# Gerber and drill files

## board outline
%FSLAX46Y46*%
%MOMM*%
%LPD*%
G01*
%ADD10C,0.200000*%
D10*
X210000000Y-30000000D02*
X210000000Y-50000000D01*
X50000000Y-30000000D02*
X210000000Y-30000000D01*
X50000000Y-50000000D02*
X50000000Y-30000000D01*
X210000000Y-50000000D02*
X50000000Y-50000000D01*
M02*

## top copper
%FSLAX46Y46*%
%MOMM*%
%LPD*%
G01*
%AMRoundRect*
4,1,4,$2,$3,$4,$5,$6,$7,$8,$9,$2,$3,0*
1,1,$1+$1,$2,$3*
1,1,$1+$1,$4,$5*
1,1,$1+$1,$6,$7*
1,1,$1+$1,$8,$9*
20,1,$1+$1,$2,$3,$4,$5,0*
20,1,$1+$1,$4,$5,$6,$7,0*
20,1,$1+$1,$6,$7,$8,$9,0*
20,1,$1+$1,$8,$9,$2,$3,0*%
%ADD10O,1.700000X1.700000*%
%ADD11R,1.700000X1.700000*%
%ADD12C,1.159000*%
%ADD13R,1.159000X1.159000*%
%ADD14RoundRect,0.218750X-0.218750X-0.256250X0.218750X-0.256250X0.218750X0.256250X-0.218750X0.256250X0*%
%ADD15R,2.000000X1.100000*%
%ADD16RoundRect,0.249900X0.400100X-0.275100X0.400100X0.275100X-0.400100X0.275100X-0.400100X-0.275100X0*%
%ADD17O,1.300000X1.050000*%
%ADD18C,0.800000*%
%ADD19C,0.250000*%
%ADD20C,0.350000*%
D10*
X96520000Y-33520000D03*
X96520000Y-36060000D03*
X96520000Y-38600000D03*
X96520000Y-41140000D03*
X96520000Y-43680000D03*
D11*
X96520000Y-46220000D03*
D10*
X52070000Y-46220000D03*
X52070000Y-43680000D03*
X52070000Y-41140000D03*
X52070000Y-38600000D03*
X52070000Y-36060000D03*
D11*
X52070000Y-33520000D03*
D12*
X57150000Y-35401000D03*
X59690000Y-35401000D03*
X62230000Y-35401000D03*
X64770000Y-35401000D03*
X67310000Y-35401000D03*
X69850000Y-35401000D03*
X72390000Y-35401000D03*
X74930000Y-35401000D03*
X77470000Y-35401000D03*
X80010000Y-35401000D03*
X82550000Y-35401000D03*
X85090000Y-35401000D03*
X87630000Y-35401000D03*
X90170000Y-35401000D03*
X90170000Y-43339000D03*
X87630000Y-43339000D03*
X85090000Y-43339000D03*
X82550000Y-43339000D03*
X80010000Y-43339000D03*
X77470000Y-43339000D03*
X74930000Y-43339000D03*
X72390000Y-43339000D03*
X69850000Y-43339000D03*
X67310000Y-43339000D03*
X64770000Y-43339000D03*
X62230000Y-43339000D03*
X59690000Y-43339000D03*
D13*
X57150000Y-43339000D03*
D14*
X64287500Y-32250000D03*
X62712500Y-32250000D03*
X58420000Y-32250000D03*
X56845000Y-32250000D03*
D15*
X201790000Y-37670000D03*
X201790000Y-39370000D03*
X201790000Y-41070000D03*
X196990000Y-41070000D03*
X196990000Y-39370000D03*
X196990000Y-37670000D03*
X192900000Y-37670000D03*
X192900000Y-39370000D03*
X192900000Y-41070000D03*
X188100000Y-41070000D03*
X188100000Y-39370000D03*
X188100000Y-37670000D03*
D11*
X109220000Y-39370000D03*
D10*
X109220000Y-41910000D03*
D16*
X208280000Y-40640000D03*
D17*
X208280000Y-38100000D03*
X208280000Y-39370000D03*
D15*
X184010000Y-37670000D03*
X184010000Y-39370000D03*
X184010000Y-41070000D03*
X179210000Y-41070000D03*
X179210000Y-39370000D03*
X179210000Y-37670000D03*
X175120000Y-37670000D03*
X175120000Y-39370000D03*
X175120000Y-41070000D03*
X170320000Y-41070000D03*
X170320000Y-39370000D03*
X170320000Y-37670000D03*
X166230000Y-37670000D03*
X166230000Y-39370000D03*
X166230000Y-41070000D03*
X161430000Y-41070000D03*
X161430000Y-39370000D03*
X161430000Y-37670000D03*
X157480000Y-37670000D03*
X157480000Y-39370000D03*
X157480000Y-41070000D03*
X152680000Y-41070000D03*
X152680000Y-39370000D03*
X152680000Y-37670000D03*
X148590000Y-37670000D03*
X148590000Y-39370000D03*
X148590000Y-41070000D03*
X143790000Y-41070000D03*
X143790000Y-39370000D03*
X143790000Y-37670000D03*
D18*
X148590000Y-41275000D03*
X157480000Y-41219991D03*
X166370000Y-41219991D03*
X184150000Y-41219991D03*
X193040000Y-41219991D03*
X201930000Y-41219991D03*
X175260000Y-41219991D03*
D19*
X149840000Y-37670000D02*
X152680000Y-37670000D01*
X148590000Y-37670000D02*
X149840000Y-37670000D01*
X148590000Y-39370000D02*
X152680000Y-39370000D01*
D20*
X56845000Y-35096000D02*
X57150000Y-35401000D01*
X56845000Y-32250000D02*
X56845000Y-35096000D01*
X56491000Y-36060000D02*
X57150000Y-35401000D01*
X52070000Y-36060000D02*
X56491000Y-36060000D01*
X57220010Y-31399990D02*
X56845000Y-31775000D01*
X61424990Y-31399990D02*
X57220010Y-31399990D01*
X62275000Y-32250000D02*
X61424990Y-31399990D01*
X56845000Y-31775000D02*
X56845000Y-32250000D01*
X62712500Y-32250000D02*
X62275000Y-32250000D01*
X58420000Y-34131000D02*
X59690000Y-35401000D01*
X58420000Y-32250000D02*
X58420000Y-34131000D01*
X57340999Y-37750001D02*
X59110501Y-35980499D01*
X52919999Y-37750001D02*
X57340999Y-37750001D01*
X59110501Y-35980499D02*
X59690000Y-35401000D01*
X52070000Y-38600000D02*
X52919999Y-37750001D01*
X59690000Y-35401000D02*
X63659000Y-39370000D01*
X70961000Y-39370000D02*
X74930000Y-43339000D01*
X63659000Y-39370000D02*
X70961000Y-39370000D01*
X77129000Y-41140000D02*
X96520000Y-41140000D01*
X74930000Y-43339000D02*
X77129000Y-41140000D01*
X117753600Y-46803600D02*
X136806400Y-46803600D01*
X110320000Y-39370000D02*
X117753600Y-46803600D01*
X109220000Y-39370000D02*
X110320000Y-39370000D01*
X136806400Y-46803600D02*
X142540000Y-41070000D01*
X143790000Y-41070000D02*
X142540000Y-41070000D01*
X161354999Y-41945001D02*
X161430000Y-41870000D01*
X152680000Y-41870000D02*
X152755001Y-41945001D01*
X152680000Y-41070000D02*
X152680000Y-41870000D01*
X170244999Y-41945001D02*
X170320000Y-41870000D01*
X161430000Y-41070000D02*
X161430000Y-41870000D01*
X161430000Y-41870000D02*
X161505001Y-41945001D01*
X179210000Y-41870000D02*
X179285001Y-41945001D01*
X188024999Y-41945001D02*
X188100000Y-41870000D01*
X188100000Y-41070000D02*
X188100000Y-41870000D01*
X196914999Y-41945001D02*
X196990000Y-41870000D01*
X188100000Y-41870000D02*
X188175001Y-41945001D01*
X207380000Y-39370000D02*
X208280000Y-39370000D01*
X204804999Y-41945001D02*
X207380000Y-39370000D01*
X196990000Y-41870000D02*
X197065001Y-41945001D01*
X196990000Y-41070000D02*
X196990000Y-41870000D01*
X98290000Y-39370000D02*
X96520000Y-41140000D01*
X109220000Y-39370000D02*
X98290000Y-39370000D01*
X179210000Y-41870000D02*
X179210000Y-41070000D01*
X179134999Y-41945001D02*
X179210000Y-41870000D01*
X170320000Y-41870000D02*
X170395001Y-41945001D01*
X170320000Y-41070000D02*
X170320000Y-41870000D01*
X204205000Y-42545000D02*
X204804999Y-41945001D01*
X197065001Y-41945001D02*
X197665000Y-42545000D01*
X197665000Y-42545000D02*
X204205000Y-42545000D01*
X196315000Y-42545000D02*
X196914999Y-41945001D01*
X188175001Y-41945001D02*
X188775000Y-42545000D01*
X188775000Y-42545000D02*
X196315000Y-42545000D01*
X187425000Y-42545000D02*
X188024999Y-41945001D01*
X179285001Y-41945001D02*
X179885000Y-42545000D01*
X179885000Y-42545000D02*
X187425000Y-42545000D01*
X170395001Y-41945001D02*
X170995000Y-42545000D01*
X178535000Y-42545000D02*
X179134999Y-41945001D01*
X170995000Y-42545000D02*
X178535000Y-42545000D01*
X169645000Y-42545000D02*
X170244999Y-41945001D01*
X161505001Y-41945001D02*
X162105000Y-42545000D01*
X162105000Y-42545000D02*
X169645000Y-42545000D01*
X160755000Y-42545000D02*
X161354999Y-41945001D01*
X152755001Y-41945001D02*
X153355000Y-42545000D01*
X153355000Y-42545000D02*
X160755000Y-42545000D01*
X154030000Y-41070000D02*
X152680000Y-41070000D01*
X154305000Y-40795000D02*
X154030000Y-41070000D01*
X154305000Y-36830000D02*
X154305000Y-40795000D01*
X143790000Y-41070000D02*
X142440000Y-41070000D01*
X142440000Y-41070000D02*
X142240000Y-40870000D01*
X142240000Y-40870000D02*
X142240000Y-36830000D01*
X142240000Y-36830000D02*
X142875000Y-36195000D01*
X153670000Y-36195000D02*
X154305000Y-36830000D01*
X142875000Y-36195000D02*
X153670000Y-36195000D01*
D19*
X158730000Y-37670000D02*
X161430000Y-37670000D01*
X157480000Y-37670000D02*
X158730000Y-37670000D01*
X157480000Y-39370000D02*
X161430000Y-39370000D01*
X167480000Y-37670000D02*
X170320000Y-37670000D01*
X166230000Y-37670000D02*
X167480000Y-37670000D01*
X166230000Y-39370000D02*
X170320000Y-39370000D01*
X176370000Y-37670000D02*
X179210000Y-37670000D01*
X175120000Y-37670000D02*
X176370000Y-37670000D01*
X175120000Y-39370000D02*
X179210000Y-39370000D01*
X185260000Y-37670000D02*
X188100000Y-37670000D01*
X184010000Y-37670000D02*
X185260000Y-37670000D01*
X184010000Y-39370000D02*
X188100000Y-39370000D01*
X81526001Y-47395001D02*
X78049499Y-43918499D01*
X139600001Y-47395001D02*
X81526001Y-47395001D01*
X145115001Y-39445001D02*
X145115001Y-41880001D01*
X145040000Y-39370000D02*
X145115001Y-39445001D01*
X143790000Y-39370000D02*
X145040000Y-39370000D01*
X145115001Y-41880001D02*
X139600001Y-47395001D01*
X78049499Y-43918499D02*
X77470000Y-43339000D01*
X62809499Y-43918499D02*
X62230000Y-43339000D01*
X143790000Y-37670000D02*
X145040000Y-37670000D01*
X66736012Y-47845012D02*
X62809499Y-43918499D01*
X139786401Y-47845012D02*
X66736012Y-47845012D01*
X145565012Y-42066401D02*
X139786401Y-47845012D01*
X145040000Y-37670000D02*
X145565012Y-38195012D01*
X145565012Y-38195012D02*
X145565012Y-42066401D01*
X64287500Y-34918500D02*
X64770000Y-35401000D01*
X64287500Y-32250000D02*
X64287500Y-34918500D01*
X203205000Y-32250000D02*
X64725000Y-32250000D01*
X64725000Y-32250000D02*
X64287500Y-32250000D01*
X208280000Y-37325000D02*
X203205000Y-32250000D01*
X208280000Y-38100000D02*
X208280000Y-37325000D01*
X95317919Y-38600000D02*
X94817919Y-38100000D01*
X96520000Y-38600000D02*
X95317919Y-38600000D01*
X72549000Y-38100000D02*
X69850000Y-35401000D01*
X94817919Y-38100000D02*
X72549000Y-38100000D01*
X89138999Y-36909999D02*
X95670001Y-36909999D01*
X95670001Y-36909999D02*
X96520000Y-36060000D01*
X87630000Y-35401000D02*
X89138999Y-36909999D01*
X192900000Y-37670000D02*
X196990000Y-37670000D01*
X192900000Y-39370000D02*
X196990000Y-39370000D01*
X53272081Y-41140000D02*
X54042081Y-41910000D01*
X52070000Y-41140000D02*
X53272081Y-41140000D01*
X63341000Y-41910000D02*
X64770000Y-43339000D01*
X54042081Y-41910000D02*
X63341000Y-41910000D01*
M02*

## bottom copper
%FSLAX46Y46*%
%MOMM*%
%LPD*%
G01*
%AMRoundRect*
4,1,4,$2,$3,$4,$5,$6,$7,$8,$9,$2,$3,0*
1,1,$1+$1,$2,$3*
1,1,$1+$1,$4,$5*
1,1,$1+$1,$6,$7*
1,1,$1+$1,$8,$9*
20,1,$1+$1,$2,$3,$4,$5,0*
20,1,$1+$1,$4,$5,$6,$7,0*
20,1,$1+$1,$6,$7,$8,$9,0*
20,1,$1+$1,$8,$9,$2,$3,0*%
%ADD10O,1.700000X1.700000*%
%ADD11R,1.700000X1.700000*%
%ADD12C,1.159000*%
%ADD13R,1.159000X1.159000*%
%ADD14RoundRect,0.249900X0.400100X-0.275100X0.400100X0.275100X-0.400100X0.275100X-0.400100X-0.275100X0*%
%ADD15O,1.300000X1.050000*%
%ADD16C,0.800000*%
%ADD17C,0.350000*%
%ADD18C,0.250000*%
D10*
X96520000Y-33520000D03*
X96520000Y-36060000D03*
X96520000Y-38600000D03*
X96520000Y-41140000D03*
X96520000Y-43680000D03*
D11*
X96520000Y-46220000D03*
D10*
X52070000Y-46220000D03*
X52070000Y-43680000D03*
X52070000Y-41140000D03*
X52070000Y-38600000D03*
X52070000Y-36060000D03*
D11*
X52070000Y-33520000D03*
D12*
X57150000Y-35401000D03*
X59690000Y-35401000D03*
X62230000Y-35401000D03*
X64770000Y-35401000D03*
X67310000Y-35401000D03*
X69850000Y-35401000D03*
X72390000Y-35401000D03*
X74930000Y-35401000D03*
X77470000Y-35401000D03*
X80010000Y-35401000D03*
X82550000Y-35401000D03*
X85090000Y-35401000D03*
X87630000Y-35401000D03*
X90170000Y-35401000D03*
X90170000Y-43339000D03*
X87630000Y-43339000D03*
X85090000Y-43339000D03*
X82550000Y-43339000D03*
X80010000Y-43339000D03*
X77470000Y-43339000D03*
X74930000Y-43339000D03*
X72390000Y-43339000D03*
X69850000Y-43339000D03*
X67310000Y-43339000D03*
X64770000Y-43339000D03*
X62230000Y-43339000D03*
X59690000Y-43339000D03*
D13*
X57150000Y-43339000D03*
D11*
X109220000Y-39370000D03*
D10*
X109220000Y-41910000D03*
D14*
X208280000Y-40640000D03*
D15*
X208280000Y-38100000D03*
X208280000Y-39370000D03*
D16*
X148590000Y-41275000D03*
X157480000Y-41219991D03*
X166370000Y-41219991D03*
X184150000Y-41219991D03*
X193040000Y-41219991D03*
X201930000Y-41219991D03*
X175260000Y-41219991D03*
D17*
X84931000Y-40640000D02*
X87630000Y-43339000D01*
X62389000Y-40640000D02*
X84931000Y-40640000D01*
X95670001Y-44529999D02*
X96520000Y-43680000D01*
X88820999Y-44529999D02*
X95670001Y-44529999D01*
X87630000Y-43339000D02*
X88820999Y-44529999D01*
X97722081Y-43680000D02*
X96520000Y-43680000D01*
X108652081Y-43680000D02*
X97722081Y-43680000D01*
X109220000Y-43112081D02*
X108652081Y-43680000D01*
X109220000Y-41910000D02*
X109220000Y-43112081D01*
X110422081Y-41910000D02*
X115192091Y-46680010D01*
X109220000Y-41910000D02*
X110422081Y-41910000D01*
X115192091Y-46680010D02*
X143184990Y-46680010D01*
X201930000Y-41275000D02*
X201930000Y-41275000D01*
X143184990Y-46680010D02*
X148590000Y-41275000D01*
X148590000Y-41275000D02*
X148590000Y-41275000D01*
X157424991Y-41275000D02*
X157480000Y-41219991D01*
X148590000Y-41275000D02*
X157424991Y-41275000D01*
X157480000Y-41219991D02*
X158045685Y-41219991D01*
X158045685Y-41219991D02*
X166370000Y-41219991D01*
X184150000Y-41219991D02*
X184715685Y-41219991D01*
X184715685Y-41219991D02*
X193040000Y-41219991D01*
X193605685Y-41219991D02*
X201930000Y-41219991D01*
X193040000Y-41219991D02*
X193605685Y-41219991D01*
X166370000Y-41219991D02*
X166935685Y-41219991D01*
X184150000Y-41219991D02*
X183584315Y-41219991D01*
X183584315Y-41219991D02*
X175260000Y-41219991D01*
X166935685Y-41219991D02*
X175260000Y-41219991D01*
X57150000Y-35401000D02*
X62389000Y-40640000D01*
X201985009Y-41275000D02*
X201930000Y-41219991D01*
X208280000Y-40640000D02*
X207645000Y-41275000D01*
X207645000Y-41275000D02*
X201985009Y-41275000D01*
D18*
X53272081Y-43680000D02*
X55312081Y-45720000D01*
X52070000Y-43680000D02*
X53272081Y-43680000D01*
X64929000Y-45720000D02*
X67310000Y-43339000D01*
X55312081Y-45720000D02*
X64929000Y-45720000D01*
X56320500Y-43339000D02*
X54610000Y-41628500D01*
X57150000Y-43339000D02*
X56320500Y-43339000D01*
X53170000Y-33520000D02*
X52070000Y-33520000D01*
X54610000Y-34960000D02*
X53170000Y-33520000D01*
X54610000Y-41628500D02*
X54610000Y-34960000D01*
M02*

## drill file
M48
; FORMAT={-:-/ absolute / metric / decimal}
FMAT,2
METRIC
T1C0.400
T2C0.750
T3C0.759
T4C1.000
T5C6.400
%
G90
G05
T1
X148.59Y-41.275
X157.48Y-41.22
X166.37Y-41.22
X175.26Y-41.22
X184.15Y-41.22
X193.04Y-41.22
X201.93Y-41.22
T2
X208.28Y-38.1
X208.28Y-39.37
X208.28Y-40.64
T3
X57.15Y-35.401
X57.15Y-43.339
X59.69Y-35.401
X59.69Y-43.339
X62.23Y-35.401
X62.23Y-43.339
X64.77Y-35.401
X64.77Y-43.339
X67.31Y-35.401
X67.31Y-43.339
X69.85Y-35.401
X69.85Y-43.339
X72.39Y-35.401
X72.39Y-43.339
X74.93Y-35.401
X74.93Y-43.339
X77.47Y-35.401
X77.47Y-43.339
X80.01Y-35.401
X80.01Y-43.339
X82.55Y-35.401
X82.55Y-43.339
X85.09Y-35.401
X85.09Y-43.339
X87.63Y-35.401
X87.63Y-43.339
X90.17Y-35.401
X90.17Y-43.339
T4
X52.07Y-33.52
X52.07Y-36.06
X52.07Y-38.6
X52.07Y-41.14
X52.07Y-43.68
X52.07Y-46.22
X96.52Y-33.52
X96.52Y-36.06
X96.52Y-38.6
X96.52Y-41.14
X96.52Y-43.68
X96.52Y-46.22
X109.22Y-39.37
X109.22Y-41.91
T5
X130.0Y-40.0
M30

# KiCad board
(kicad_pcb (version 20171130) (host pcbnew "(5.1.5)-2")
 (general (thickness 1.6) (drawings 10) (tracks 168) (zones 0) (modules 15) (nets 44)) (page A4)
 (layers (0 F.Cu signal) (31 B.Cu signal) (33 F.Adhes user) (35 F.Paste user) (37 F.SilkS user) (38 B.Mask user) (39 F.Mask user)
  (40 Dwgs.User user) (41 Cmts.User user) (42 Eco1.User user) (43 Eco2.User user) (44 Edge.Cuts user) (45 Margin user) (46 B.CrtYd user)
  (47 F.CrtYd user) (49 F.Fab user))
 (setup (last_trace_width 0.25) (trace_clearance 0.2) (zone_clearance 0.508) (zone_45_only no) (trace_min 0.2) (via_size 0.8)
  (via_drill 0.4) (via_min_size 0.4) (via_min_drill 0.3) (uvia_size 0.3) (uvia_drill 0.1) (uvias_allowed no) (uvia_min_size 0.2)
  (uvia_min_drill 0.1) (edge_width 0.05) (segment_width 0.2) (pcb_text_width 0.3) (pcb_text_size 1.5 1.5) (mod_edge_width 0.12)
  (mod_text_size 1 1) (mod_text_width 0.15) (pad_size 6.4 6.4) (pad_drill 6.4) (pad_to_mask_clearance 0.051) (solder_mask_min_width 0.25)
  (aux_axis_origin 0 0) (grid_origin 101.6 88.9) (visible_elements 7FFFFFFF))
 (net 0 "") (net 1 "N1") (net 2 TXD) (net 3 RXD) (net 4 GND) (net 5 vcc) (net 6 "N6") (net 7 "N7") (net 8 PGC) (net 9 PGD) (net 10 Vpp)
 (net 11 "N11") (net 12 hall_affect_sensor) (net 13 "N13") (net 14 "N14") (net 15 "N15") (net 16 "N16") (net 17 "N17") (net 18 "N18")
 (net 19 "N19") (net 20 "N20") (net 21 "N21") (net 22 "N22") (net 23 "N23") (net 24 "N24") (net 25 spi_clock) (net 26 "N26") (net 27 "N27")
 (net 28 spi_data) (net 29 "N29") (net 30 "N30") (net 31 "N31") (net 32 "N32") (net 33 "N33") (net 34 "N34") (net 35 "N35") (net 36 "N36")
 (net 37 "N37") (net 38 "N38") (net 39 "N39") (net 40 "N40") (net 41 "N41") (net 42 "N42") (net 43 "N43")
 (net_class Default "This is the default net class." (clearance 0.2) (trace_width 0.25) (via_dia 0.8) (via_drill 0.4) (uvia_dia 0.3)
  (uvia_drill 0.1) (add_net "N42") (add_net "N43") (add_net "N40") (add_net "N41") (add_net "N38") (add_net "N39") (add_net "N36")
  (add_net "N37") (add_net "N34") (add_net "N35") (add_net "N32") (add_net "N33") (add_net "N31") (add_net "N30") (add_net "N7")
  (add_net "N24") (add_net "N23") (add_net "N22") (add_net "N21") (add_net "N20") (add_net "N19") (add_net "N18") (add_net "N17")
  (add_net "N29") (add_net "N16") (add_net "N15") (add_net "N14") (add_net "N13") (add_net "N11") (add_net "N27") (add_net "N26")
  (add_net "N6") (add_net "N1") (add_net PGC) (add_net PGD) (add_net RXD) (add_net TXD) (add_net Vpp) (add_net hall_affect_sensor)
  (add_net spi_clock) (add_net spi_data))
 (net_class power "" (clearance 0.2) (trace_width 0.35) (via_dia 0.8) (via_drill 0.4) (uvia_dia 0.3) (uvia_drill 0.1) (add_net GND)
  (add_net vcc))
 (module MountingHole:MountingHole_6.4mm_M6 (layer F.Cu) (at 130 40)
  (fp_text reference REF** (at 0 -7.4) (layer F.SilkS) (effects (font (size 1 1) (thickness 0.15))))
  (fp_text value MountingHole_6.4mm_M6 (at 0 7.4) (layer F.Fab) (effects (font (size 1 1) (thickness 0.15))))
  (pad 1 np_thru_hole circle (at 0 0) (size 6.4 6.4) (drill 6.4) (layers *.Cu *.Mask)))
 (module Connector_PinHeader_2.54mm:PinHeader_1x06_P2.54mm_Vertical (layer F.Cu) (at 96.52 46.22 180)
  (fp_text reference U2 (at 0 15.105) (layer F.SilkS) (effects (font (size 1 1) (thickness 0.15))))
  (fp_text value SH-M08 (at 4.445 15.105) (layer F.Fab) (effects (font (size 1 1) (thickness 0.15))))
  (pad 6 thru_hole oval (at 0 12.7 180) (size 1.7 1.7) (drill 1) (layers *.Cu *.Mask) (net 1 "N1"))
  (pad 5 thru_hole oval (at 0 10.16 180) (size 1.7 1.7) (drill 1) (layers *.Cu *.Mask) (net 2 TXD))
  (pad 4 thru_hole oval (at 0 7.62 180) (size 1.7 1.7) (drill 1) (layers *.Cu *.Mask) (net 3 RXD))
  (pad 3 thru_hole oval (at 0 5.08 180) (size 1.7 1.7) (drill 1) (layers *.Cu *.Mask) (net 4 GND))
  (pad 2 thru_hole oval (at 0 2.54 180) (size 1.7 1.7) (drill 1) (layers *.Cu *.Mask) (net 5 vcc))
  (pad 1 thru_hole rect (at 0 0 180) (size 1.7 1.7) (drill 1) (layers *.Cu *.Mask) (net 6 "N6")))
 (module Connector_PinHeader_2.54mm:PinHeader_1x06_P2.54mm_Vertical (layer F.Cu) (at 52.07 33.52)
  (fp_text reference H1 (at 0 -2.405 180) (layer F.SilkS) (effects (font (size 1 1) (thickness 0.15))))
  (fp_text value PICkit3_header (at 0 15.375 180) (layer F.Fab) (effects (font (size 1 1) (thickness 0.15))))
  (pad 6 thru_hole oval (at 0 12.7) (size 1.7 1.7) (drill 1) (layers *.Cu *.Mask) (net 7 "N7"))
  (pad 5 thru_hole oval (at 0 10.16) (size 1.7 1.7) (drill 1) (layers *.Cu *.Mask) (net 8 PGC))
  (pad 4 thru_hole oval (at 0 7.62) (size 1.7 1.7) (drill 1) (layers *.Cu *.Mask) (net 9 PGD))
  (pad 3 thru_hole oval (at 0 5.08) (size 1.7 1.7) (drill 1) (layers *.Cu *.Mask) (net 4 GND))
  (pad 2 thru_hole oval (at 0 2.54) (size 1.7 1.7) (drill 1) (layers *.Cu *.Mask) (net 5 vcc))
  (pad 1 thru_hole rect (at 0 0) (size 1.7 1.7) (drill 1) (layers *.Cu *.Mask) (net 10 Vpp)))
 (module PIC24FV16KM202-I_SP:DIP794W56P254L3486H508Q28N (layer F.Cu) (at 73.66 39.37 90)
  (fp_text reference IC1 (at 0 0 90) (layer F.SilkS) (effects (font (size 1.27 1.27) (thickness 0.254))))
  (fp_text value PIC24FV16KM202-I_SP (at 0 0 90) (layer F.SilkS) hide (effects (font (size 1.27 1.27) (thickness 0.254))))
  (pad 28 thru_hole circle (at 3.969 -16.51 180) (size 1.159 1.159) (drill 0.759) (layers *.Cu *.Mask) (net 5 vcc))
  (pad 27 thru_hole circle (at 3.969 -13.97 180) (size 1.159 1.159) (drill 0.759) (layers *.Cu *.Mask) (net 4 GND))
  (pad 26 thru_hole circle (at 3.969 -11.43 180) (size 1.159 1.159) (drill 0.759) (layers *.Cu *.Mask) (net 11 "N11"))
  (pad 25 thru_hole circle (at 3.969 -8.89 180) (size 1.159 1.159) (drill 0.759) (layers *.Cu *.Mask) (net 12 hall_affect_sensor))
  (pad 24 thru_hole circle (at 3.969 -6.35 180) (size 1.159 1.159) (drill 0.759) (layers *.Cu *.Mask) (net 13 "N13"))
  (pad 23 thru_hole circle (at 3.969 -3.81 180) (size 1.159 1.159) (drill 0.759) (layers *.Cu *.Mask) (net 3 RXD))
  (pad 22 thru_hole circle (at 3.969 -1.27 180) (size 1.159 1.159) (drill 0.759) (layers *.Cu *.Mask) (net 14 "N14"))
  (pad 21 thru_hole circle (at 3.969 1.27 180) (size 1.159 1.159) (drill 0.759) (layers *.Cu *.Mask) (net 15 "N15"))
  (pad 20 thru_hole circle (at 3.969 3.81 180) (size 1.159 1.159) (drill 0.759) (layers *.Cu *.Mask) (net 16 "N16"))
  (pad 19 thru_hole circle (at 3.969 6.35 180) (size 1.159 1.159) (drill 0.759) (layers *.Cu *.Mask) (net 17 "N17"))
  (pad 18 thru_hole circle (at 3.969 8.89 180) (size 1.159 1.159) (drill 0.759) (layers *.Cu *.Mask) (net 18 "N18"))
  (pad 17 thru_hole circle (at 3.969 11.43 180) (size 1.159 1.159) (drill 0.759) (layers *.Cu *.Mask) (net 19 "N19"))
  (pad 16 thru_hole circle (at 3.969 13.97 180) (size 1.159 1.159) (drill 0.759) (layers *.Cu *.Mask) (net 2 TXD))
  (pad 15 thru_hole circle (at 3.969 16.51 180) (size 1.159 1.159) (drill 0.759) (layers *.Cu *.Mask) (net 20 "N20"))
  (pad 14 thru_hole circle (at -3.969 16.51 180) (size 1.159 1.159) (drill 0.759) (layers *.Cu *.Mask) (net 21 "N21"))
  (pad 13 thru_hole circle (at -3.969 13.97 180) (size 1.159 1.159) (drill 0.759) (layers *.Cu *.Mask) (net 5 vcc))
  (pad 12 thru_hole circle (at -3.969 11.43 180) (size 1.159 1.159) (drill 0.759) (layers *.Cu *.Mask) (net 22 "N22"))
  (pad 11 thru_hole circle (at -3.969 8.89 180) (size 1.159 1.159) (drill 0.759) (layers *.Cu *.Mask) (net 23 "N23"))
  (pad 10 thru_hole circle (at -3.969 6.35 180) (size 1.159 1.159) (drill 0.759) (layers *.Cu *.Mask) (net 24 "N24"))
  (pad 9 thru_hole circle (at -3.969 3.81 180) (size 1.159 1.159) (drill 0.759) (layers *.Cu *.Mask) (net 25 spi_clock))
  (pad 8 thru_hole circle (at -3.969 1.27 180) (size 1.159 1.159) (drill 0.759) (layers *.Cu *.Mask) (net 4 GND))
  (pad 7 thru_hole circle (at -3.969 -1.27 180) (size 1.159 1.159) (drill 0.759) (layers *.Cu *.Mask) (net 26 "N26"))
  (pad 6 thru_hole circle (at -3.969 -3.81 180) (size 1.159 1.159) (drill 0.759) (layers *.Cu *.Mask) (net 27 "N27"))
  (pad 5 thru_hole circle (at -3.969 -6.35 180) (size 1.159 1.159) (drill 0.759) (layers *.Cu *.Mask) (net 8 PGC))
  (pad 4 thru_hole circle (at -3.969 -8.89 180) (size 1.159 1.159) (drill 0.759) (layers *.Cu *.Mask) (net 9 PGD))
  (pad 3 thru_hole circle (at -3.969 -11.43 180) (size 1.159 1.159) (drill 0.759) (layers *.Cu *.Mask) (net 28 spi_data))
  (pad 2 thru_hole circle (at -3.969 -13.97 180) (size 1.159 1.159) (drill 0.759) (layers *.Cu *.Mask) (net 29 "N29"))
  (pad 1 thru_hole rect (at -3.969 -16.51 180) (size 1.159 1.159) (drill 0.759) (layers *.Cu *.Mask) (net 10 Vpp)))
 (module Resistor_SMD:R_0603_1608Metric (layer F.Cu) (at 63.5 32.25)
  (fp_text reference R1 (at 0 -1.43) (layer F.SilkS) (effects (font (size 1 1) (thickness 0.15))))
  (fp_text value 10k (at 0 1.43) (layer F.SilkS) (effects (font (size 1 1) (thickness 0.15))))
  (pad 2 smd roundrect (at 0.7875 0) (size 0.875 0.95) (layers F.Cu F.Paste F.Mask) (roundrect_rratio 0.25) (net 12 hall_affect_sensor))
  (pad 1 smd roundrect (at -0.7875 0) (size 0.875 0.95) (layers F.Cu F.Paste F.Mask) (roundrect_rratio 0.25) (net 5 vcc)))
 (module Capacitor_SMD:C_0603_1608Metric (layer F.Cu) (at 57.6325 32.25)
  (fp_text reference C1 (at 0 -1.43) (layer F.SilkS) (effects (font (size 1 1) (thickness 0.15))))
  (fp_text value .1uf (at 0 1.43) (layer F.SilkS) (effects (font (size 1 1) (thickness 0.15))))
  (pad 2 smd roundrect (at 0.7875 0) (size 0.875 0.95) (layers F.Cu F.Paste F.Mask) (roundrect_rratio 0.25) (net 4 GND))
  (pad 1 smd roundrect (at -0.7875 0) (size 0.875 0.95) (layers F.Cu F.Paste F.Mask) (roundrect_rratio 0.25) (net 5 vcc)))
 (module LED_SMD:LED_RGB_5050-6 (layer F.Cu) (at 199.39 39.37)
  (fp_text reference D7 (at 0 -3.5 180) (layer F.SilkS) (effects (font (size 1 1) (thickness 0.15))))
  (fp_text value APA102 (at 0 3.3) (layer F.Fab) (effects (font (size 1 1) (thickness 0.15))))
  (pad 6 smd rect (at 2.4 -1.7 90) (size 1.1 2) (layers F.Cu F.Paste F.Mask) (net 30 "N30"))
  (pad 5 smd rect (at 2.4 0 90) (size 1.1 2) (layers F.Cu F.Paste F.Mask) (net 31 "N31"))
  (pad 4 smd rect (at 2.4 1.7 90) (size 1.1 2) (layers F.Cu F.Paste F.Mask) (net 5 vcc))
  (pad 3 smd rect (at -2.4 1.7 90) (size 1.1 2) (layers F.Cu F.Paste F.Mask) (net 4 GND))
  (pad 2 smd rect (at -2.4 0 90) (size 1.1 2) (layers F.Cu F.Paste F.Mask) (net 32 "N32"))
  (pad 1 smd rect (at -2.4 -1.7 90) (size 1.1 2) (layers F.Cu F.Paste F.Mask) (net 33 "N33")))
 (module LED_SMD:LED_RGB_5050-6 (layer F.Cu) (at 190.5 39.37)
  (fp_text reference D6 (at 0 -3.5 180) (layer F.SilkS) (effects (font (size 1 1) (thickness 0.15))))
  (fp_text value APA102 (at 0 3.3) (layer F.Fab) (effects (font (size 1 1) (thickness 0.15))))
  (pad 6 smd rect (at 2.4 -1.7 90) (size 1.1 2) (layers F.Cu F.Paste F.Mask) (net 33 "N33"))
  (pad 5 smd rect (at 2.4 0 90) (size 1.1 2) (layers F.Cu F.Paste F.Mask) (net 32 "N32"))
  (pad 4 smd rect (at 2.4 1.7 90) (size 1.1 2) (layers F.Cu F.Paste F.Mask) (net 5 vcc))
  (pad 3 smd rect (at -2.4 1.7 90) (size 1.1 2) (layers F.Cu F.Paste F.Mask) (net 4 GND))
  (pad 2 smd rect (at -2.4 0 90) (size 1.1 2) (layers F.Cu F.Paste F.Mask) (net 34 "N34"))
  (pad 1 smd rect (at -2.4 -1.7 90) (size 1.1 2) (layers F.Cu F.Paste F.Mask) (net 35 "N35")))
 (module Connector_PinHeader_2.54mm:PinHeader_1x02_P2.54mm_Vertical (layer F.Cu) (at 109.22 39.37)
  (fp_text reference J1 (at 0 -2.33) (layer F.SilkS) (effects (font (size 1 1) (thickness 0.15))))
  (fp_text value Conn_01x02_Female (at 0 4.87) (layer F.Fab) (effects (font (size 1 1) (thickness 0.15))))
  (pad 1 thru_hole rect (at 0 0) (size 1.7 1.7) (drill 1) (layers *.Cu *.Mask) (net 4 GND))
  (pad 2 thru_hole oval (at 0 2.54) (size 1.7 1.7) (drill 1) (layers *.Cu *.Mask) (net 5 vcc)))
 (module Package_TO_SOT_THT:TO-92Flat (layer F.Cu) (at 208.28 40.64 90)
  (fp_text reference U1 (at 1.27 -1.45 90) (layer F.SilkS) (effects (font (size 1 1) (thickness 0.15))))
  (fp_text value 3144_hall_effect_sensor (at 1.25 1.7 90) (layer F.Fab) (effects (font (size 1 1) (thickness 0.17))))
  (pad 1 thru_hole roundrect (at 0 0 90) (size 1.05 1.3) (drill 0.75) (layers *.Cu *.Mask) (roundrect_rratio 0.238) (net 5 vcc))
  (pad 3 thru_hole oval (at 2.54 0 90) (size 1.05 1.3) (drill 0.75) (layers *.Cu *.Mask) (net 12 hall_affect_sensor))
  (pad 2 thru_hole oval (at 1.27 0 90) (size 1.05 1.3) (drill 0.75) (layers *.Cu *.Mask) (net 4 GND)))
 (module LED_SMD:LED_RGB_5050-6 (layer F.Cu) (at 181.61 39.37)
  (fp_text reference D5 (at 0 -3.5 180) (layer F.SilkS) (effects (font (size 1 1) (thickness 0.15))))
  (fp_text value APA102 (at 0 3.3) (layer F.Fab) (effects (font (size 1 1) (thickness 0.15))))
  (pad 6 smd rect (at 2.4 -1.7 90) (size 1.1 2) (layers F.Cu F.Paste F.Mask) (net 35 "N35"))
  (pad 5 smd rect (at 2.4 0 90) (size 1.1 2) (layers F.Cu F.Paste F.Mask) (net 34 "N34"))
  (pad 4 smd rect (at 2.4 1.7 90) (size 1.1 2) (layers F.Cu F.Paste F.Mask) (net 5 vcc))
  (pad 3 smd rect (at -2.4 1.7 90) (size 1.1 2) (layers F.Cu F.Paste F.Mask) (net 4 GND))
  (pad 2 smd rect (at -2.4 0 90) (size 1.1 2) (layers F.Cu F.Paste F.Mask) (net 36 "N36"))
  (pad 1 smd rect (at -2.4 -1.7 90) (size 1.1 2) (layers F.Cu F.Paste F.Mask) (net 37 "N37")))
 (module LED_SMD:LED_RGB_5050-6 (layer F.Cu) (at 172.72 39.37)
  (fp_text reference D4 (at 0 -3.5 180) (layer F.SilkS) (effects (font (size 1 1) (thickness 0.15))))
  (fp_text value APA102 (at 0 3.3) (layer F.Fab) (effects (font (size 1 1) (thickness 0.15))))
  (pad 6 smd rect (at 2.4 -1.7 90) (size 1.1 2) (layers F.Cu F.Paste F.Mask) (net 37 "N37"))
  (pad 5 smd rect (at 2.4 0 90) (size 1.1 2) (layers F.Cu F.Paste F.Mask) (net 36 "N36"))
  (pad 4 smd rect (at 2.4 1.7 90) (size 1.1 2) (layers F.Cu F.Paste F.Mask) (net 5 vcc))
  (pad 3 smd rect (at -2.4 1.7 90) (size 1.1 2) (layers F.Cu F.Paste F.Mask) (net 4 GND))
  (pad 2 smd rect (at -2.4 0 90) (size 1.1 2) (layers F.Cu F.Paste F.Mask) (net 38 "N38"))
  (pad 1 smd rect (at -2.4 -1.7 90) (size 1.1 2) (layers F.Cu F.Paste F.Mask) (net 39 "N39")))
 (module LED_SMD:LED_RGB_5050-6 (layer F.Cu) (at 163.83 39.37)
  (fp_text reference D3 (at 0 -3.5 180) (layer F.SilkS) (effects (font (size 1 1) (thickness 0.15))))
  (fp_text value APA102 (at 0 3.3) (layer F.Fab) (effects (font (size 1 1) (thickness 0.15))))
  (pad 6 smd rect (at 2.4 -1.7 90) (size 1.1 2) (layers F.Cu F.Paste F.Mask) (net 39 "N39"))
  (pad 5 smd rect (at 2.4 0 90) (size 1.1 2) (layers F.Cu F.Paste F.Mask) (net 38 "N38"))
  (pad 4 smd rect (at 2.4 1.7 90) (size 1.1 2) (layers F.Cu F.Paste F.Mask) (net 5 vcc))
  (pad 3 smd rect (at -2.4 1.7 90) (size 1.1 2) (layers F.Cu F.Paste F.Mask) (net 4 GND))
  (pad 2 smd rect (at -2.4 0 90) (size 1.1 2) (layers F.Cu F.Paste F.Mask) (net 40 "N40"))
  (pad 1 smd rect (at -2.4 -1.7 90) (size 1.1 2) (layers F.Cu F.Paste F.Mask) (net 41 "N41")))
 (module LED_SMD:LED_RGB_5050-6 (layer F.Cu) (at 155.08 39.37)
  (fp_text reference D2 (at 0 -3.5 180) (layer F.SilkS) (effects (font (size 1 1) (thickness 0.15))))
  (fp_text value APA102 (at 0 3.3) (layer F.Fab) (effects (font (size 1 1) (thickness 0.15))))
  (pad 6 smd rect (at 2.4 -1.7 90) (size 1.1 2) (layers F.Cu F.Paste F.Mask) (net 41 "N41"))
  (pad 5 smd rect (at 2.4 0 90) (size 1.1 2) (layers F.Cu F.Paste F.Mask) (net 40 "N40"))
  (pad 4 smd rect (at 2.4 1.7 90) (size 1.1 2) (layers F.Cu F.Paste F.Mask) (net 5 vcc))
  (pad 3 smd rect (at -2.4 1.7 90) (size 1.1 2) (layers F.Cu F.Paste F.Mask) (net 4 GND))
  (pad 2 smd rect (at -2.4 0 90) (size 1.1 2) (layers F.Cu F.Paste F.Mask) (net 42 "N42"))
  (pad 1 smd rect (at -2.4 -1.7 90) (size 1.1 2) (layers F.Cu F.Paste F.Mask) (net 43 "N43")))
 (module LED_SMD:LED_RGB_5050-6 (layer F.Cu) (at 146.19 39.37)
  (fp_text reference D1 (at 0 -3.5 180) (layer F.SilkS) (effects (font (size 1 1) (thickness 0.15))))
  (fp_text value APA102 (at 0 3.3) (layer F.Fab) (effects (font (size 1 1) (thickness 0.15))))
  (pad 6 smd rect (at 2.4 -1.7 90) (size 1.1 2) (layers F.Cu F.Paste F.Mask) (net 43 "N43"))
  (pad 5 smd rect (at 2.4 0 90) (size 1.1 2) (layers F.Cu F.Paste F.Mask) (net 42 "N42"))
  (pad 4 smd rect (at 2.4 1.7 90) (size 1.1 2) (layers F.Cu F.Paste F.Mask) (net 5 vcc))
  (pad 3 smd rect (at -2.4 1.7 90) (size 1.1 2) (layers F.Cu F.Paste F.Mask) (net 4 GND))
  (pad 2 smd rect (at -2.4 0 90) (size 1.1 2) (layers F.Cu F.Paste F.Mask) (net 25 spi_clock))
  (pad 1 smd rect (at -2.4 -1.7 90) (size 1.1 2) (layers F.Cu F.Paste F.Mask) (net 28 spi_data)))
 (gr_line (start 210 30) (end 210 50) (layer Edge.Cuts) (width 0.2))
 (gr_line (start 50 30) (end 210 30) (layer Edge.Cuts) (width 0.2))
 (gr_line (start 50 50) (end 50 30) (layer Edge.Cuts) (width 0.2))
 (gr_line (start 210 50) (end 50 50) (layer Edge.Cuts) (width 0.2))
 (segment (start 149.84 37.67) (end 152.68 37.67) (width 0.25) (layer F.Cu) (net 43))
 (segment (start 148.59 37.67) (end 149.84 37.67) (width 0.25) (layer F.Cu) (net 43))
 (segment (start 148.59 39.37) (end 152.68 39.37) (width 0.25) (layer F.Cu) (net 42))
 (segment (start 56.845 35.096) (end 57.15 35.401) (width 0.35) (layer F.Cu) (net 5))
 (segment (start 56.845 32.25) (end 56.845 35.096) (width 0.35) (layer F.Cu) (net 5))
 (segment (start 56.491 36.06) (end 57.15 35.401) (width 0.35) (layer F.Cu) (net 5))
 (segment (start 52.07 36.06) (end 56.491 36.06) (width 0.35) (layer F.Cu) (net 5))
 (segment (start 84.931 40.64) (end 87.63 43.339) (width 0.35) (layer B.Cu) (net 5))
 (segment (start 62.389 40.64) (end 84.931 40.64) (width 0.35) (layer B.Cu) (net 5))
 (segment (start 95.670001 44.529999) (end 96.52 43.68) (width 0.35) (layer B.Cu) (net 5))
 (segment (start 88.820999 44.529999) (end 95.670001 44.529999) (width 0.35) (layer B.Cu) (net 5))
 (segment (start 87.63 43.339) (end 88.820999 44.529999) (width 0.35) (layer B.Cu) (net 5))
 (segment (start 97.722081 43.68) (end 96.52 43.68) (width 0.35) (layer B.Cu) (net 5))
 (segment (start 108.652081 43.68) (end 97.722081 43.68) (width 0.35) (layer B.Cu) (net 5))
 (segment (start 109.22 43.112081) (end 108.652081 43.68) (width 0.35) (layer B.Cu) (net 5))
 (segment (start 109.22 41.91) (end 109.22 43.112081) (width 0.35) (layer B.Cu) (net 5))
 (segment (start 110.422081 41.91) (end 115.192091 46.68001) (width 0.35) (layer B.Cu) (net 5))
 (segment (start 109.22 41.91) (end 110.422081 41.91) (width 0.35) (layer B.Cu) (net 5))
 (segment (start 115.192091 46.68001) (end 143.18499 46.68001) (width 0.35) (layer B.Cu) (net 5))
 (segment (start 201.93 41.275) (end 201.93 41.275) (width 0.35) (layer B.Cu) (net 5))
 (segment (start 143.18499 46.68001) (end 148.59 41.275) (width 0.35) (layer B.Cu) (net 5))
 (segment (start 148.59 41.275) (end 148.59 41.275) (width 0.35) (layer B.Cu) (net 5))
 (via (at 148.59 41.275) (size 0.8) (drill 0.4) (layers F.Cu B.Cu) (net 5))
 (via (at 157.48 41.219991) (size 0.8) (drill 0.4) (layers F.Cu B.Cu) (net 5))
 (segment (start 157.424991 41.275) (end 157.48 41.219991) (width 0.35) (layer B.Cu) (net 5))
 (segment (start 148.59 41.275) (end 157.424991 41.275) (width 0.35) (layer B.Cu) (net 5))
 (segment (start 157.48 41.219991) (end 158.045685 41.219991) (width 0.35) (layer B.Cu) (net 5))
 (segment (start 158.045685 41.219991) (end 166.37 41.219991) (width 0.35) (layer B.Cu) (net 5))
 (via (at 166.37 41.219991) (size 0.8) (drill 0.4) (layers F.Cu B.Cu) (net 5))
 (via (at 184.15 41.219991) (size 0.8) (drill 0.4) (layers F.Cu B.Cu) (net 5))
 (segment (start 184.15 41.219991) (end 184.715685 41.219991) (width 0.35) (layer B.Cu) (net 5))
 (segment (start 184.715685 41.219991) (end 193.04 41.219991) (width 0.35) (layer B.Cu) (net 5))
 (via (at 193.04 41.219991) (size 0.8) (drill 0.4) (layers F.Cu B.Cu) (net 5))
 (via (at 201.93 41.219991) (size 0.8) (drill 0.4) (layers F.Cu B.Cu) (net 5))
 (segment (start 193.605685 41.219991) (end 201.93 41.219991) (width 0.35) (layer B.Cu) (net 5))
 (segment (start 193.04 41.219991) (end 193.605685 41.219991) (width 0.35) (layer B.Cu) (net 5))
 (segment (start 166.37 41.219991) (end 166.935685 41.219991) (width 0.35) (layer B.Cu) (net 5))
 (segment (start 184.15 41.219991) (end 183.584315 41.219991) (width 0.35) (layer B.Cu) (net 5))
 (segment (start 183.584315 41.219991) (end 175.26 41.219991) (width 0.35) (layer B.Cu) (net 5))
 (segment (start 166.935685 41.219991) (end 175.26 41.219991) (width 0.35) (layer B.Cu) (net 5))
 (via (at 175.26 41.219991) (size 0.8) (drill 0.4) (layers F.Cu B.Cu) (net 5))
 (segment (start 57.15 35.401) (end 62.389 40.64) (width 0.35) (layer B.Cu) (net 5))
 (segment (start 201.985009 41.275) (end 201.93 41.219991) (width 0.35) (layer B.Cu) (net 5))
 (segment (start 208.28 40.64) (end 207.645 41.275) (width 0.35) (layer B.Cu) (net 5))
 (segment (start 207.645 41.275) (end 201.985009 41.275) (width 0.35) (layer B.Cu) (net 5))
 (segment (start 57.22001 31.39999) (end 56.845 31.775) (width 0.35) (layer F.Cu) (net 5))
 (segment (start 61.42499 31.39999) (end 57.22001 31.39999) (width 0.35) (layer F.Cu) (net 5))
 (segment (start 62.275 32.25) (end 61.42499 31.39999) (width 0.35) (layer F.Cu) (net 5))
 (segment (start 56.845 31.775) (end 56.845 32.25) (width 0.35) (layer F.Cu) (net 5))
 (segment (start 62.7125 32.25) (end 62.275 32.25) (width 0.35) (layer F.Cu) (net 5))
 (segment (start 58.42 34.131) (end 59.69 35.401) (width 0.35) (layer F.Cu) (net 4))
 (segment (start 58.42 32.25) (end 58.42 34.131) (width 0.35) (layer F.Cu) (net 4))
 (segment (start 57.340999 37.750001) (end 59.110501 35.980499) (width 0.35) (layer F.Cu) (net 4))
 (segment (start 52.919999 37.750001) (end 57.340999 37.750001) (width 0.35) (layer F.Cu) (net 4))
 (segment (start 59.110501 35.980499) (end 59.69 35.401) (width 0.35) (layer F.Cu) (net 4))
 (segment (start 52.07 38.6) (end 52.919999 37.750001) (width 0.35) (layer F.Cu) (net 4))
 (segment (start 59.69 35.401) (end 63.659 39.37) (width 0.35) (layer F.Cu) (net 4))
 (segment (start 70.961 39.37) (end 74.93 43.339) (width 0.35) (layer F.Cu) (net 4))
 (segment (start 63.659 39.37) (end 70.961 39.37) (width 0.35) (layer F.Cu) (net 4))
 (segment (start 77.129 41.14) (end 96.52 41.14) (width 0.35) (layer F.Cu) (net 4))
 (segment (start 74.93 43.339) (end 77.129 41.14) (width 0.35) (layer F.Cu) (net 4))
 (segment (start 117.7536 46.8036) (end 136.8064 46.8036) (width 0.35) (layer F.Cu) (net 4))
 (segment (start 110.32 39.37) (end 117.7536 46.8036) (width 0.35) (layer F.Cu) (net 4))
 (segment (start 109.22 39.37) (end 110.32 39.37) (width 0.35) (layer F.Cu) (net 4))
 (segment (start 136.8064 46.8036) (end 142.54 41.07) (width 0.35) (layer F.Cu) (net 4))
 (segment (start 143.79 41.07) (end 142.54 41.07) (width 0.35) (layer F.Cu) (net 4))
 (segment (start 161.354999 41.945001) (end 161.43 41.87) (width 0.35) (layer F.Cu) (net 4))
 (segment (start 152.68 41.87) (end 152.755001 41.945001) (width 0.35) (layer F.Cu) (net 4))
 (segment (start 152.68 41.07) (end 152.68 41.87) (width 0.35) (layer F.Cu) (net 4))
 (segment (start 170.244999 41.945001) (end 170.32 41.87) (width 0.35) (layer F.Cu) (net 4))
 (segment (start 161.43 41.07) (end 161.43 41.87) (width 0.35) (layer F.Cu) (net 4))
 (segment (start 161.43 41.87) (end 161.505001 41.945001) (width 0.35) (layer F.Cu) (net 4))
 (segment (start 179.21 41.87) (end 179.285001 41.945001) (width 0.35) (layer F.Cu) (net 4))
 (segment (start 188.024999 41.945001) (end 188.1 41.87) (width 0.35) (layer F.Cu) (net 4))
 (segment (start 188.1 41.07) (end 188.1 41.87) (width 0.35) (layer F.Cu) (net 4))
 (segment (start 196.914999 41.945001) (end 196.99 41.87) (width 0.35) (layer F.Cu) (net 4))
 (segment (start 188.1 41.87) (end 188.175001 41.945001) (width 0.35) (layer F.Cu) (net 4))
 (segment (start 207.38 39.37) (end 208.28 39.37) (width 0.35) (layer F.Cu) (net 4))
 (segment (start 204.804999 41.945001) (end 207.38 39.37) (width 0.35) (layer F.Cu) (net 4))
 (segment (start 196.99 41.87) (end 197.065001 41.945001) (width 0.35) (layer F.Cu) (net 4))
 (segment (start 196.99 41.07) (end 196.99 41.87) (width 0.35) (layer F.Cu) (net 4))
 (segment (start 98.29 39.37) (end 96.52 41.14) (width 0.35) (layer F.Cu) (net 4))
 (segment (start 109.22 39.37) (end 98.29 39.37) (width 0.35) (layer F.Cu) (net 4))
 (segment (start 179.21 41.87) (end 179.21 41.07) (width 0.35) (layer F.Cu) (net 4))
 (segment (start 179.134999 41.945001) (end 179.21 41.87) (width 0.35) (layer F.Cu) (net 4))
 (segment (start 170.32 41.87) (end 170.395001 41.945001) (width 0.35) (layer F.Cu) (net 4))
 (segment (start 170.32 41.07) (end 170.32 41.87) (width 0.35) (layer F.Cu) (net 4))
 (segment (start 204.205 42.545) (end 204.804999 41.945001) (width 0.35) (layer F.Cu) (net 4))
 (segment (start 197.065001 41.945001) (end 197.665 42.545) (width 0.35) (layer F.Cu) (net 4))
 (segment (start 197.665 42.545) (end 204.205 42.545) (width 0.35) (layer F.Cu) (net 4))
 (segment (start 196.315 42.545) (end 196.914999 41.945001) (width 0.35) (layer F.Cu) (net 4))
 (segment (start 188.175001 41.945001) (end 188.775 42.545) (width 0.35) (layer F.Cu) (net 4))
 (segment (start 188.775 42.545) (end 196.315 42.545) (width 0.35) (layer F.Cu) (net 4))
 (segment (start 187.425 42.545) (end 188.024999 41.945001) (width 0.35) (layer F.Cu) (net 4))
 (segment (start 179.285001 41.945001) (end 179.885 42.545) (width 0.35) (layer F.Cu) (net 4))
 (segment (start 179.885 42.545) (end 187.425 42.545) (width 0.35) (layer F.Cu) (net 4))
 (segment (start 170.395001 41.945001) (end 170.995 42.545) (width 0.35) (layer F.Cu) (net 4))
 (segment (start 178.535 42.545) (end 179.134999 41.945001) (width 0.35) (layer F.Cu) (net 4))
 (segment (start 170.995 42.545) (end 178.535 42.545) (width 0.35) (layer F.Cu) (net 4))
 (segment (start 169.645 42.545) (end 170.244999 41.945001) (width 0.35) (layer F.Cu) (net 4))
 (segment (start 161.505001 41.945001) (end 162.105 42.545) (width 0.35) (layer F.Cu) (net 4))
 (segment (start 162.105 42.545) (end 169.645 42.545) (width 0.35) (layer F.Cu) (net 4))
 (segment (start 160.755 42.545) (end 161.354999 41.945001) (width 0.35) (layer F.Cu) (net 4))
 (segment (start 152.755001 41.945001) (end 153.355 42.545) (width 0.35) (layer F.Cu) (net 4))
 (segment (start 153.355 42.545) (end 160.755 42.545) (width 0.35) (layer F.Cu) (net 4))
 (segment (start 154.03 41.07) (end 152.68 41.07) (width 0.35) (layer F.Cu) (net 4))
 (segment (start 154.305 40.795) (end 154.03 41.07) (width 0.35) (layer F.Cu) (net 4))
 (segment (start 154.305 36.83) (end 154.305 40.795) (width 0.35) (layer F.Cu) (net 4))
 (segment (start 143.79 41.07) (end 142.44 41.07) (width 0.35) (layer F.Cu) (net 4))
 (segment (start 142.44 41.07) (end 142.24 40.87) (width 0.35) (layer F.Cu) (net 4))
 (segment (start 142.24 40.87) (end 142.24 36.83) (width 0.35) (layer F.Cu) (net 4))
 (segment (start 142.24 36.83) (end 142.875 36.195) (width 0.35) (layer F.Cu) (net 4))
 (segment (start 153.67 36.195) (end 154.305 36.83) (width 0.35) (layer F.Cu) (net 4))
 (segment (start 142.875 36.195) (end 153.67 36.195) (width 0.35) (layer F.Cu) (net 4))
 (segment (start 158.73 37.67) (end 161.43 37.67) (width 0.25) (layer F.Cu) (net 41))
 (segment (start 157.48 37.67) (end 158.73 37.67) (width 0.25) (layer F.Cu) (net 41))
 (segment (start 157.48 39.37) (end 161.43 39.37) (width 0.25) (layer F.Cu) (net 40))
 (segment (start 167.48 37.67) (end 170.32 37.67) (width 0.25) (layer F.Cu) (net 39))
 (segment (start 166.23 37.67) (end 167.48 37.67) (width 0.25) (layer F.Cu) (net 39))
 (segment (start 166.23 39.37) (end 170.32 39.37) (width 0.25) (layer F.Cu) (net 38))
 (segment (start 176.37 37.67) (end 179.21 37.67) (width 0.25) (layer F.Cu) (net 37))
 (segment (start 175.12 37.67) (end 176.37 37.67) (width 0.25) (layer F.Cu) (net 37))
 (segment (start 175.12 39.37) (end 179.21 39.37) (width 0.25) (layer F.Cu) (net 36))
 (segment (start 185.26 37.67) (end 188.1 37.67) (width 0.25) (layer F.Cu) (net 35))
 (segment (start 184.01 37.67) (end 185.26 37.67) (width 0.25) (layer F.Cu) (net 35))
 (segment (start 184.01 39.37) (end 188.1 39.37) (width 0.25) (layer F.Cu) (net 34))
 (segment (start 81.526001 47.395001) (end 78.049499 43.918499) (width 0.25) (layer F.Cu) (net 25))
 (segment (start 139.600001 47.395001) (end 81.526001 47.395001) (width 0.25) (layer F.Cu) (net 25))
 (segment (start 145.115001 39.445001) (end 145.115001 41.880001) (width 0.25) (layer F.Cu) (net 25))
 (segment (start 145.04 39.37) (end 145.115001 39.445001) (width 0.25) (layer F.Cu) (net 25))
 (segment (start 143.79 39.37) (end 145.04 39.37) (width 0.25) (layer F.Cu) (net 25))
 (segment (start 145.115001 41.880001) (end 139.600001 47.395001) (width 0.25) (layer F.Cu) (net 25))
 (segment (start 78.049499 43.918499) (end 77.47 43.339) (width 0.25) (layer F.Cu) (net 25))
 (segment (start 62.809499 43.918499) (end 62.23 43.339) (width 0.25) (layer F.Cu) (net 28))
 (segment (start 143.79 37.67) (end 145.04 37.67) (width 0.25) (layer F.Cu) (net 28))
 (segment (start 66.736012 47.845012) (end 62.809499 43.918499) (width 0.25) (layer F.Cu) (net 28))
 (segment (start 139.786401 47.845012) (end 66.736012 47.845012) (width 0.25) (layer F.Cu) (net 28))
 (segment (start 145.565012 42.066401) (end 139.786401 47.845012) (width 0.25) (layer F.Cu) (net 28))
 (segment (start 145.04 37.67) (end 145.565012 38.195012) (width 0.25) (layer F.Cu) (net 28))
 (segment (start 145.565012 38.195012) (end 145.565012 42.066401) (width 0.25) (layer F.Cu) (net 28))
 (segment (start 64.2875 34.9185) (end 64.77 35.401) (width 0.25) (layer F.Cu) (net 12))
 (segment (start 64.2875 32.25) (end 64.2875 34.9185) (width 0.25) (layer F.Cu) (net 12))
 (segment (start 203.205 32.25) (end 64.725 32.25) (width 0.25) (layer F.Cu) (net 12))
 (segment (start 64.725 32.25) (end 64.2875 32.25) (width 0.25) (layer F.Cu) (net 12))
 (segment (start 208.28 37.325) (end 203.205 32.25) (width 0.25) (layer F.Cu) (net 12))
 (segment (start 208.28 38.1) (end 208.28 37.325) (width 0.25) (layer F.Cu) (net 12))
 (segment (start 95.317919 38.6) (end 94.817919 38.1) (width 0.25) (layer F.Cu) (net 3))
 (segment (start 96.52 38.6) (end 95.317919 38.6) (width 0.25) (layer F.Cu) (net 3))
 (segment (start 72.549 38.1) (end 69.85 35.401) (width 0.25) (layer F.Cu) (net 3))
 (segment (start 94.817919 38.1) (end 72.549 38.1) (width 0.25) (layer F.Cu) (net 3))
 (segment (start 89.138999 36.909999) (end 95.670001 36.909999) (width 0.25) (layer F.Cu) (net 2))
 (segment (start 95.670001 36.909999) (end 96.52 36.06) (width 0.25) (layer F.Cu) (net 2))
 (segment (start 87.63 35.401) (end 89.138999 36.909999) (width 0.25) (layer F.Cu) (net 2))
 (segment (start 192.9 37.67) (end 196.99 37.67) (width 0.25) (layer F.Cu) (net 33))
 (segment (start 192.9 39.37) (end 196.99 39.37) (width 0.25) (layer F.Cu) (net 32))
 (segment (start 53.272081 43.68) (end 55.312081 45.72) (width 0.25) (layer B.Cu) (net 8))
 (segment (start 52.07 43.68) (end 53.272081 43.68) (width 0.25) (layer B.Cu) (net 8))
 (segment (start 64.929 45.72) (end 67.31 43.339) (width 0.25) (layer B.Cu) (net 8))
 (segment (start 55.312081 45.72) (end 64.929 45.72) (width 0.25) (layer B.Cu) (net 8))
 (segment (start 53.272081 41.14) (end 54.042081 41.91) (width 0.25) (layer F.Cu) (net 9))
 (segment (start 52.07 41.14) (end 53.272081 41.14) (width 0.25) (layer F.Cu) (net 9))
 (segment (start 63.341 41.91) (end 64.77 43.339) (width 0.25) (layer F.Cu) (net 9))
 (segment (start 54.042081 41.91) (end 63.341 41.91) (width 0.25) (layer F.Cu) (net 9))
 (segment (start 56.3205 43.339) (end 54.61 41.6285) (width 0.25) (layer B.Cu) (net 10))
 (segment (start 57.15 43.339) (end 56.3205 43.339) (width 0.25) (layer B.Cu) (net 10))
 (segment (start 53.17 33.52) (end 52.07 33.52) (width 0.25) (layer B.Cu) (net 10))
 (segment (start 54.61 34.96) (end 53.17 33.52) (width 0.25) (layer B.Cu) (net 10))
 (segment (start 54.61 41.6285) (end 54.61 34.96) (width 0.25) (layer B.Cu) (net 10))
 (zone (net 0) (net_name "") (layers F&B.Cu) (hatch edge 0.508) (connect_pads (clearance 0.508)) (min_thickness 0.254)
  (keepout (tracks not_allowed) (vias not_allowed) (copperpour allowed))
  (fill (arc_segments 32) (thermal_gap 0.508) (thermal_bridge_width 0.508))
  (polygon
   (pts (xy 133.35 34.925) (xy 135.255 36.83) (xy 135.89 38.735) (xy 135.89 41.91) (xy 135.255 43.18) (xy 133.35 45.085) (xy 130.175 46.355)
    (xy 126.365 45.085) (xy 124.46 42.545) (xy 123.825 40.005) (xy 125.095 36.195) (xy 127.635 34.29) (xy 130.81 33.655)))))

